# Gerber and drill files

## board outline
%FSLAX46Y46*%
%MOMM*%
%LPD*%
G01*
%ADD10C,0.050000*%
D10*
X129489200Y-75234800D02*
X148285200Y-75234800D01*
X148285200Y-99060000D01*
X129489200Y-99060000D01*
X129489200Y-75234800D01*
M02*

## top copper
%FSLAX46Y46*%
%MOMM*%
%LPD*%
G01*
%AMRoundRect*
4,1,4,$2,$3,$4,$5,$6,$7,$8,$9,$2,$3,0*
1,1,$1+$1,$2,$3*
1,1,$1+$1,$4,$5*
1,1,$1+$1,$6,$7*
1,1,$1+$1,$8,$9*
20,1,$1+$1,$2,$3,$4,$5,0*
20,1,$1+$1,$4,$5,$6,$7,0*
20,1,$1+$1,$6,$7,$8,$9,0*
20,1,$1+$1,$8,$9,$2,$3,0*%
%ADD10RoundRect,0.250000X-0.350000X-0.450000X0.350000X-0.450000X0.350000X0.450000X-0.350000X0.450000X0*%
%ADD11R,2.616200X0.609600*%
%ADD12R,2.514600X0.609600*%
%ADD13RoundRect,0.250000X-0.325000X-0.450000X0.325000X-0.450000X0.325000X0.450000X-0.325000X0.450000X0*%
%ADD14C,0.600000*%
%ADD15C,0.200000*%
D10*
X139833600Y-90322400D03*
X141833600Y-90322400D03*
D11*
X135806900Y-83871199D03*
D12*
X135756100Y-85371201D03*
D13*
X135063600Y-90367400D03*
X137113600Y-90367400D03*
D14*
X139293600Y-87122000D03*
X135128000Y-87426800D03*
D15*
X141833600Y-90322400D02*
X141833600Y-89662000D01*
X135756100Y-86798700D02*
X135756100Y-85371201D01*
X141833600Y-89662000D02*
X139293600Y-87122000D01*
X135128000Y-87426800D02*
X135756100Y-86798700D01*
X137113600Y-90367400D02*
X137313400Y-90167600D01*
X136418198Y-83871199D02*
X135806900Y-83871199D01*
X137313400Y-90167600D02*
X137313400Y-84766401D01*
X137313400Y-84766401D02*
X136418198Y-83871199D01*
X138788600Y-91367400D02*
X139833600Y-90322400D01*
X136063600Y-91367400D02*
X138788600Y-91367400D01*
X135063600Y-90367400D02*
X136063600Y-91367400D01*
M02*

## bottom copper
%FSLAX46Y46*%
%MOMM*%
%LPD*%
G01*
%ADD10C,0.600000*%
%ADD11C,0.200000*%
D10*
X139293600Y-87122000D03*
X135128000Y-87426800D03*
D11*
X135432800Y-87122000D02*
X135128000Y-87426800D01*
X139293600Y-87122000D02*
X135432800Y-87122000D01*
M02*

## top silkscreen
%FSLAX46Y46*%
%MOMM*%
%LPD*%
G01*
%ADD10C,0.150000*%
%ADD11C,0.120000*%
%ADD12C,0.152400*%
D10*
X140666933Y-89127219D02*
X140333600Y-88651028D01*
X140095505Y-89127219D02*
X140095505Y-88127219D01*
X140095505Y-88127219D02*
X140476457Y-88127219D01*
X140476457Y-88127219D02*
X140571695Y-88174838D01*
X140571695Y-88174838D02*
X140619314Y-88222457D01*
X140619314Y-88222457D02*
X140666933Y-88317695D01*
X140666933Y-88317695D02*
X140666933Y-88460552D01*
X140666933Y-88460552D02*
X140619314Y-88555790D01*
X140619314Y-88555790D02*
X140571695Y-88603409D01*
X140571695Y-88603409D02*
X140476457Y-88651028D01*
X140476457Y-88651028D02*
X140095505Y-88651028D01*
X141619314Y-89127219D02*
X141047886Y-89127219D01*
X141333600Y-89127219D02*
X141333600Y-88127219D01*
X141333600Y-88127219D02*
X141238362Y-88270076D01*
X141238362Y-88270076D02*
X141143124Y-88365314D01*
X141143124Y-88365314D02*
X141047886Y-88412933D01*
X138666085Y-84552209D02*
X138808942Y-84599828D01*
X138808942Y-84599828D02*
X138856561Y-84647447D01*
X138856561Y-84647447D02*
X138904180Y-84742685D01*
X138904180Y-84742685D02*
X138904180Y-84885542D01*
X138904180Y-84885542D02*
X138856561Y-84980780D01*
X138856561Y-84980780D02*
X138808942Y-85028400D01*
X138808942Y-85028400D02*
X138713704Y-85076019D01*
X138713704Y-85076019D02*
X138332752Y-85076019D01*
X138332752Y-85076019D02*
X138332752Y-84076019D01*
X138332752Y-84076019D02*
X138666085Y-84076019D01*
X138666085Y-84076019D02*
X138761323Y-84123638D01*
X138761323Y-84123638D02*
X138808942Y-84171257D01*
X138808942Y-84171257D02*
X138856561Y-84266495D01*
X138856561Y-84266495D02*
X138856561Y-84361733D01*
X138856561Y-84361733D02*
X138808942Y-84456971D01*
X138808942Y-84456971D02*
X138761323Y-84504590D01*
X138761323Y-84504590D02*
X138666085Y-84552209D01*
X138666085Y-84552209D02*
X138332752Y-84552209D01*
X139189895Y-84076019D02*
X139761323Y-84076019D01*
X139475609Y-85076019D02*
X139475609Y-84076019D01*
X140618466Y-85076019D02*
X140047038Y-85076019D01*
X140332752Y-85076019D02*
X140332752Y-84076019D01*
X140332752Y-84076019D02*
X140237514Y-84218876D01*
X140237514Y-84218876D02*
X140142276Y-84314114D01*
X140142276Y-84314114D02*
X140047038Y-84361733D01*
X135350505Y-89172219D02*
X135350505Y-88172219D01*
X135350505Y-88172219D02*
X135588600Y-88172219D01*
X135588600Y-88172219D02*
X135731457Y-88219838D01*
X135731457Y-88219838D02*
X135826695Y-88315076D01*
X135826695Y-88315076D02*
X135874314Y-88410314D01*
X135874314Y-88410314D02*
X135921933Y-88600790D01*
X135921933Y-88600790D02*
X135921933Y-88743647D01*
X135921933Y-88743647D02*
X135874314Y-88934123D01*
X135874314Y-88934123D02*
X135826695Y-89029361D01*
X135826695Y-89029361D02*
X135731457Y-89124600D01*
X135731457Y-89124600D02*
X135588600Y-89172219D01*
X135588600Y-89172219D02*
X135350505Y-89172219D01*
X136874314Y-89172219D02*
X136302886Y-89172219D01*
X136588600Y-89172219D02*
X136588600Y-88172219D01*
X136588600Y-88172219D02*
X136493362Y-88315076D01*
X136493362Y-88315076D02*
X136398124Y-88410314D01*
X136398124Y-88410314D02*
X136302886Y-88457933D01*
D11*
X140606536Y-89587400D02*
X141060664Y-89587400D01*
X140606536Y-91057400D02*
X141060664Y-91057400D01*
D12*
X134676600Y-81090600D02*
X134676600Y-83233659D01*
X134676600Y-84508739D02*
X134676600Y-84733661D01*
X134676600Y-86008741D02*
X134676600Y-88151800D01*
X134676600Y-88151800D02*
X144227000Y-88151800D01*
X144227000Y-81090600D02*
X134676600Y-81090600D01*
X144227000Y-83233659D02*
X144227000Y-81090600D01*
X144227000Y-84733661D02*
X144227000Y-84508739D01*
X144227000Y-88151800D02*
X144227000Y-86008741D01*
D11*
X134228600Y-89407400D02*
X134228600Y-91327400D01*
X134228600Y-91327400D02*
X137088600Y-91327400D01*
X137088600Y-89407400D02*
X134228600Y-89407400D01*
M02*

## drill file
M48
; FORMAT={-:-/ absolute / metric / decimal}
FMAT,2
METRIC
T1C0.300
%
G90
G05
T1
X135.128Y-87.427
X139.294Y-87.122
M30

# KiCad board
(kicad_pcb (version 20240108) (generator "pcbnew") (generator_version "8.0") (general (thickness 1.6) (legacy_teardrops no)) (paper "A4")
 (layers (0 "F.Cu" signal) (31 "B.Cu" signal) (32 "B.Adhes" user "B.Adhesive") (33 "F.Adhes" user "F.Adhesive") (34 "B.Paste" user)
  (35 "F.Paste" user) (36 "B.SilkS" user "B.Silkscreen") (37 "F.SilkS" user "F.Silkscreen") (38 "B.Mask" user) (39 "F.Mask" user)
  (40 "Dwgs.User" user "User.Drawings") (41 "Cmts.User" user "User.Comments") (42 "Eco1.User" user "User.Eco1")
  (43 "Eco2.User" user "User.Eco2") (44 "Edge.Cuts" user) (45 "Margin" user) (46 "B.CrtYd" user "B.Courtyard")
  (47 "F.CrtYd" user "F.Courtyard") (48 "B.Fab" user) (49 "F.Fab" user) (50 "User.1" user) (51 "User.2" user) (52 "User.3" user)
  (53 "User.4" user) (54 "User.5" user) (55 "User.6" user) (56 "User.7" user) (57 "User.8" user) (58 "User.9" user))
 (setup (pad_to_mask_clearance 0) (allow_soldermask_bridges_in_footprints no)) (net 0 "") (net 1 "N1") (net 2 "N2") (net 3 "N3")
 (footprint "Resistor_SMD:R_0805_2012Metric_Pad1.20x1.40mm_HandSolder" (layer "F.Cu") (at 140.8336 90.3224)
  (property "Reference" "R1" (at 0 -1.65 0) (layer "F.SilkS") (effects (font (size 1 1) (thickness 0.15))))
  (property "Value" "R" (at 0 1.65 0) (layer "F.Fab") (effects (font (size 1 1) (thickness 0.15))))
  (fp_line (start -0.227064 -0.735) (end 0.227064 -0.735) (stroke (width 0.12) (type solid)) (layer "F.SilkS"))
  (fp_line (start -0.227064 0.735) (end 0.227064 0.735) (stroke (width 0.12) (type solid)) (layer "F.SilkS"))
  (pad "1" smd roundrect (at -1 0) (size 1.2 1.4) (layers "F.Cu" "F.Paste" "F.Mask") (roundrect_rratio 0.208333) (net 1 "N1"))
  (pad "2" smd roundrect (at 1 0) (size 1.2 1.4) (layers "F.Cu" "F.Paste" "F.Mask") (roundrect_rratio 0.208333) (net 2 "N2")))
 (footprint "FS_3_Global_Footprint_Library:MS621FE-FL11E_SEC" (layer "F.Cu") (at 139.4518 84.6212)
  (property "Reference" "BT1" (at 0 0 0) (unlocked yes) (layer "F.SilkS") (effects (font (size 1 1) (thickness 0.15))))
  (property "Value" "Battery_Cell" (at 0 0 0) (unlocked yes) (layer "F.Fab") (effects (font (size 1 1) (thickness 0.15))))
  (fp_line (start -4.7752 -3.5306) (end -4.7752 -1.387541) (stroke (width 0.1524) (type solid)) (layer "F.SilkS"))
  (fp_line (start -4.7752 -0.112461) (end -4.7752 0.112461) (stroke (width 0.1524) (type solid)) (layer "F.SilkS"))
  (fp_line (start -4.7752 1.387541) (end -4.7752 3.5306) (stroke (width 0.1524) (type solid)) (layer "F.SilkS"))
  (fp_line (start -4.7752 3.5306) (end 4.7752 3.5306) (stroke (width 0.1524) (type solid)) (layer "F.SilkS"))
  (fp_line (start 4.7752 -3.5306) (end -4.7752 -3.5306) (stroke (width 0.1524) (type solid)) (layer "F.SilkS"))
  (fp_line (start 4.7752 -1.387541) (end 4.7752 -3.5306) (stroke (width 0.1524) (type solid)) (layer "F.SilkS"))
  (fp_line (start 4.7752 0.112461) (end 4.7752 -0.112461) (stroke (width 0.1524) (type solid)) (layer "F.SilkS"))
  (fp_line (start 4.7752 3.5306) (end 4.7752 1.387541) (stroke (width 0.1524) (type solid)) (layer "F.SilkS"))
  (pad "1" smd rect (at -3.6449 -0.750001) (size 2.6162 0.6096) (layers "F.Cu" "F.Paste" "F.Mask") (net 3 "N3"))
  (pad "2" smd rect (at -3.6957 0.750001) (size 2.5146 0.6096) (layers "F.Cu" "F.Paste" "F.Mask") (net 2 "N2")))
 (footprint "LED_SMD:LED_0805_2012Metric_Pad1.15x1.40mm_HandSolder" (layer "F.Cu") (at 136.0886 90.3674)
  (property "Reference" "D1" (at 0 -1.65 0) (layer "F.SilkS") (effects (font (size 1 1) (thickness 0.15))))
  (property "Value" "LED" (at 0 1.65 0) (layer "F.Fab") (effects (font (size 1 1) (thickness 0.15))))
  (fp_line (start -1.86 -0.96) (end -1.86 0.96) (stroke (width 0.12) (type solid)) (layer "F.SilkS"))
  (fp_line (start -1.86 0.96) (end 1 0.96) (stroke (width 0.12) (type solid)) (layer "F.SilkS"))
  (fp_line (start 1 -0.96) (end -1.86 -0.96) (stroke (width 0.12) (type solid)) (layer "F.SilkS"))
  (pad "1" smd roundrect (at -1.025 0) (size 1.15 1.4) (layers "F.Cu" "F.Paste" "F.Mask") (roundrect_rratio 0.217391) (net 1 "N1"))
  (pad "2" smd roundrect (at 1.025 0) (size 1.15 1.4) (layers "F.Cu" "F.Paste" "F.Mask") (roundrect_rratio 0.217391) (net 3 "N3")))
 (gr_rect (start 129.4892 75.2348) (end 148.2852 99.06) (stroke (width 0.05) (type default)) (fill none) (layer "Edge.Cuts"))
 (segment (start 141.8336 90.3224) (end 141.8336 89.662) (width 0.2) (layer "F.Cu") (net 2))
 (segment (start 135.7561 86.7987) (end 135.7561 85.371201) (width 0.2) (layer "F.Cu") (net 2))
 (segment (start 141.8336 89.662) (end 139.2936 87.122) (width 0.2) (layer "F.Cu") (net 2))
 (segment (start 135.128 87.4268) (end 135.7561 86.7987) (width 0.2) (layer "F.Cu") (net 2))
 (via (at 139.2936 87.122) (size 0.6) (drill 0.3) (layers "F.Cu" "B.Cu") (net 2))
 (via (at 135.128 87.4268) (size 0.6) (drill 0.3) (layers "F.Cu" "B.Cu") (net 2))
 (segment (start 135.4328 87.122) (end 135.128 87.4268) (width 0.2) (layer "B.Cu") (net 2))
 (segment (start 139.2936 87.122) (end 135.4328 87.122) (width 0.2) (layer "B.Cu") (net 2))
 (segment (start 137.1136 90.3674) (end 137.3134 90.1676) (width 0.2) (layer "F.Cu") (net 3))
 (segment (start 136.418198 83.871199) (end 135.8069 83.871199) (width 0.2) (layer "F.Cu") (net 3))
 (segment (start 137.3134 90.1676) (end 137.3134 84.766401) (width 0.2) (layer "F.Cu") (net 3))
 (segment (start 137.3134 84.766401) (end 136.418198 83.871199) (width 0.2) (layer "F.Cu") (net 3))
 (segment (start 138.7886 91.3674) (end 139.8336 90.3224) (width 0.2) (layer "F.Cu") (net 1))
 (segment (start 136.0636 91.3674) (end 138.7886 91.3674) (width 0.2) (layer "F.Cu") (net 1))
 (segment (start 135.0636 90.3674) (end 136.0636 91.3674) (width 0.2) (layer "F.Cu") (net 1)))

